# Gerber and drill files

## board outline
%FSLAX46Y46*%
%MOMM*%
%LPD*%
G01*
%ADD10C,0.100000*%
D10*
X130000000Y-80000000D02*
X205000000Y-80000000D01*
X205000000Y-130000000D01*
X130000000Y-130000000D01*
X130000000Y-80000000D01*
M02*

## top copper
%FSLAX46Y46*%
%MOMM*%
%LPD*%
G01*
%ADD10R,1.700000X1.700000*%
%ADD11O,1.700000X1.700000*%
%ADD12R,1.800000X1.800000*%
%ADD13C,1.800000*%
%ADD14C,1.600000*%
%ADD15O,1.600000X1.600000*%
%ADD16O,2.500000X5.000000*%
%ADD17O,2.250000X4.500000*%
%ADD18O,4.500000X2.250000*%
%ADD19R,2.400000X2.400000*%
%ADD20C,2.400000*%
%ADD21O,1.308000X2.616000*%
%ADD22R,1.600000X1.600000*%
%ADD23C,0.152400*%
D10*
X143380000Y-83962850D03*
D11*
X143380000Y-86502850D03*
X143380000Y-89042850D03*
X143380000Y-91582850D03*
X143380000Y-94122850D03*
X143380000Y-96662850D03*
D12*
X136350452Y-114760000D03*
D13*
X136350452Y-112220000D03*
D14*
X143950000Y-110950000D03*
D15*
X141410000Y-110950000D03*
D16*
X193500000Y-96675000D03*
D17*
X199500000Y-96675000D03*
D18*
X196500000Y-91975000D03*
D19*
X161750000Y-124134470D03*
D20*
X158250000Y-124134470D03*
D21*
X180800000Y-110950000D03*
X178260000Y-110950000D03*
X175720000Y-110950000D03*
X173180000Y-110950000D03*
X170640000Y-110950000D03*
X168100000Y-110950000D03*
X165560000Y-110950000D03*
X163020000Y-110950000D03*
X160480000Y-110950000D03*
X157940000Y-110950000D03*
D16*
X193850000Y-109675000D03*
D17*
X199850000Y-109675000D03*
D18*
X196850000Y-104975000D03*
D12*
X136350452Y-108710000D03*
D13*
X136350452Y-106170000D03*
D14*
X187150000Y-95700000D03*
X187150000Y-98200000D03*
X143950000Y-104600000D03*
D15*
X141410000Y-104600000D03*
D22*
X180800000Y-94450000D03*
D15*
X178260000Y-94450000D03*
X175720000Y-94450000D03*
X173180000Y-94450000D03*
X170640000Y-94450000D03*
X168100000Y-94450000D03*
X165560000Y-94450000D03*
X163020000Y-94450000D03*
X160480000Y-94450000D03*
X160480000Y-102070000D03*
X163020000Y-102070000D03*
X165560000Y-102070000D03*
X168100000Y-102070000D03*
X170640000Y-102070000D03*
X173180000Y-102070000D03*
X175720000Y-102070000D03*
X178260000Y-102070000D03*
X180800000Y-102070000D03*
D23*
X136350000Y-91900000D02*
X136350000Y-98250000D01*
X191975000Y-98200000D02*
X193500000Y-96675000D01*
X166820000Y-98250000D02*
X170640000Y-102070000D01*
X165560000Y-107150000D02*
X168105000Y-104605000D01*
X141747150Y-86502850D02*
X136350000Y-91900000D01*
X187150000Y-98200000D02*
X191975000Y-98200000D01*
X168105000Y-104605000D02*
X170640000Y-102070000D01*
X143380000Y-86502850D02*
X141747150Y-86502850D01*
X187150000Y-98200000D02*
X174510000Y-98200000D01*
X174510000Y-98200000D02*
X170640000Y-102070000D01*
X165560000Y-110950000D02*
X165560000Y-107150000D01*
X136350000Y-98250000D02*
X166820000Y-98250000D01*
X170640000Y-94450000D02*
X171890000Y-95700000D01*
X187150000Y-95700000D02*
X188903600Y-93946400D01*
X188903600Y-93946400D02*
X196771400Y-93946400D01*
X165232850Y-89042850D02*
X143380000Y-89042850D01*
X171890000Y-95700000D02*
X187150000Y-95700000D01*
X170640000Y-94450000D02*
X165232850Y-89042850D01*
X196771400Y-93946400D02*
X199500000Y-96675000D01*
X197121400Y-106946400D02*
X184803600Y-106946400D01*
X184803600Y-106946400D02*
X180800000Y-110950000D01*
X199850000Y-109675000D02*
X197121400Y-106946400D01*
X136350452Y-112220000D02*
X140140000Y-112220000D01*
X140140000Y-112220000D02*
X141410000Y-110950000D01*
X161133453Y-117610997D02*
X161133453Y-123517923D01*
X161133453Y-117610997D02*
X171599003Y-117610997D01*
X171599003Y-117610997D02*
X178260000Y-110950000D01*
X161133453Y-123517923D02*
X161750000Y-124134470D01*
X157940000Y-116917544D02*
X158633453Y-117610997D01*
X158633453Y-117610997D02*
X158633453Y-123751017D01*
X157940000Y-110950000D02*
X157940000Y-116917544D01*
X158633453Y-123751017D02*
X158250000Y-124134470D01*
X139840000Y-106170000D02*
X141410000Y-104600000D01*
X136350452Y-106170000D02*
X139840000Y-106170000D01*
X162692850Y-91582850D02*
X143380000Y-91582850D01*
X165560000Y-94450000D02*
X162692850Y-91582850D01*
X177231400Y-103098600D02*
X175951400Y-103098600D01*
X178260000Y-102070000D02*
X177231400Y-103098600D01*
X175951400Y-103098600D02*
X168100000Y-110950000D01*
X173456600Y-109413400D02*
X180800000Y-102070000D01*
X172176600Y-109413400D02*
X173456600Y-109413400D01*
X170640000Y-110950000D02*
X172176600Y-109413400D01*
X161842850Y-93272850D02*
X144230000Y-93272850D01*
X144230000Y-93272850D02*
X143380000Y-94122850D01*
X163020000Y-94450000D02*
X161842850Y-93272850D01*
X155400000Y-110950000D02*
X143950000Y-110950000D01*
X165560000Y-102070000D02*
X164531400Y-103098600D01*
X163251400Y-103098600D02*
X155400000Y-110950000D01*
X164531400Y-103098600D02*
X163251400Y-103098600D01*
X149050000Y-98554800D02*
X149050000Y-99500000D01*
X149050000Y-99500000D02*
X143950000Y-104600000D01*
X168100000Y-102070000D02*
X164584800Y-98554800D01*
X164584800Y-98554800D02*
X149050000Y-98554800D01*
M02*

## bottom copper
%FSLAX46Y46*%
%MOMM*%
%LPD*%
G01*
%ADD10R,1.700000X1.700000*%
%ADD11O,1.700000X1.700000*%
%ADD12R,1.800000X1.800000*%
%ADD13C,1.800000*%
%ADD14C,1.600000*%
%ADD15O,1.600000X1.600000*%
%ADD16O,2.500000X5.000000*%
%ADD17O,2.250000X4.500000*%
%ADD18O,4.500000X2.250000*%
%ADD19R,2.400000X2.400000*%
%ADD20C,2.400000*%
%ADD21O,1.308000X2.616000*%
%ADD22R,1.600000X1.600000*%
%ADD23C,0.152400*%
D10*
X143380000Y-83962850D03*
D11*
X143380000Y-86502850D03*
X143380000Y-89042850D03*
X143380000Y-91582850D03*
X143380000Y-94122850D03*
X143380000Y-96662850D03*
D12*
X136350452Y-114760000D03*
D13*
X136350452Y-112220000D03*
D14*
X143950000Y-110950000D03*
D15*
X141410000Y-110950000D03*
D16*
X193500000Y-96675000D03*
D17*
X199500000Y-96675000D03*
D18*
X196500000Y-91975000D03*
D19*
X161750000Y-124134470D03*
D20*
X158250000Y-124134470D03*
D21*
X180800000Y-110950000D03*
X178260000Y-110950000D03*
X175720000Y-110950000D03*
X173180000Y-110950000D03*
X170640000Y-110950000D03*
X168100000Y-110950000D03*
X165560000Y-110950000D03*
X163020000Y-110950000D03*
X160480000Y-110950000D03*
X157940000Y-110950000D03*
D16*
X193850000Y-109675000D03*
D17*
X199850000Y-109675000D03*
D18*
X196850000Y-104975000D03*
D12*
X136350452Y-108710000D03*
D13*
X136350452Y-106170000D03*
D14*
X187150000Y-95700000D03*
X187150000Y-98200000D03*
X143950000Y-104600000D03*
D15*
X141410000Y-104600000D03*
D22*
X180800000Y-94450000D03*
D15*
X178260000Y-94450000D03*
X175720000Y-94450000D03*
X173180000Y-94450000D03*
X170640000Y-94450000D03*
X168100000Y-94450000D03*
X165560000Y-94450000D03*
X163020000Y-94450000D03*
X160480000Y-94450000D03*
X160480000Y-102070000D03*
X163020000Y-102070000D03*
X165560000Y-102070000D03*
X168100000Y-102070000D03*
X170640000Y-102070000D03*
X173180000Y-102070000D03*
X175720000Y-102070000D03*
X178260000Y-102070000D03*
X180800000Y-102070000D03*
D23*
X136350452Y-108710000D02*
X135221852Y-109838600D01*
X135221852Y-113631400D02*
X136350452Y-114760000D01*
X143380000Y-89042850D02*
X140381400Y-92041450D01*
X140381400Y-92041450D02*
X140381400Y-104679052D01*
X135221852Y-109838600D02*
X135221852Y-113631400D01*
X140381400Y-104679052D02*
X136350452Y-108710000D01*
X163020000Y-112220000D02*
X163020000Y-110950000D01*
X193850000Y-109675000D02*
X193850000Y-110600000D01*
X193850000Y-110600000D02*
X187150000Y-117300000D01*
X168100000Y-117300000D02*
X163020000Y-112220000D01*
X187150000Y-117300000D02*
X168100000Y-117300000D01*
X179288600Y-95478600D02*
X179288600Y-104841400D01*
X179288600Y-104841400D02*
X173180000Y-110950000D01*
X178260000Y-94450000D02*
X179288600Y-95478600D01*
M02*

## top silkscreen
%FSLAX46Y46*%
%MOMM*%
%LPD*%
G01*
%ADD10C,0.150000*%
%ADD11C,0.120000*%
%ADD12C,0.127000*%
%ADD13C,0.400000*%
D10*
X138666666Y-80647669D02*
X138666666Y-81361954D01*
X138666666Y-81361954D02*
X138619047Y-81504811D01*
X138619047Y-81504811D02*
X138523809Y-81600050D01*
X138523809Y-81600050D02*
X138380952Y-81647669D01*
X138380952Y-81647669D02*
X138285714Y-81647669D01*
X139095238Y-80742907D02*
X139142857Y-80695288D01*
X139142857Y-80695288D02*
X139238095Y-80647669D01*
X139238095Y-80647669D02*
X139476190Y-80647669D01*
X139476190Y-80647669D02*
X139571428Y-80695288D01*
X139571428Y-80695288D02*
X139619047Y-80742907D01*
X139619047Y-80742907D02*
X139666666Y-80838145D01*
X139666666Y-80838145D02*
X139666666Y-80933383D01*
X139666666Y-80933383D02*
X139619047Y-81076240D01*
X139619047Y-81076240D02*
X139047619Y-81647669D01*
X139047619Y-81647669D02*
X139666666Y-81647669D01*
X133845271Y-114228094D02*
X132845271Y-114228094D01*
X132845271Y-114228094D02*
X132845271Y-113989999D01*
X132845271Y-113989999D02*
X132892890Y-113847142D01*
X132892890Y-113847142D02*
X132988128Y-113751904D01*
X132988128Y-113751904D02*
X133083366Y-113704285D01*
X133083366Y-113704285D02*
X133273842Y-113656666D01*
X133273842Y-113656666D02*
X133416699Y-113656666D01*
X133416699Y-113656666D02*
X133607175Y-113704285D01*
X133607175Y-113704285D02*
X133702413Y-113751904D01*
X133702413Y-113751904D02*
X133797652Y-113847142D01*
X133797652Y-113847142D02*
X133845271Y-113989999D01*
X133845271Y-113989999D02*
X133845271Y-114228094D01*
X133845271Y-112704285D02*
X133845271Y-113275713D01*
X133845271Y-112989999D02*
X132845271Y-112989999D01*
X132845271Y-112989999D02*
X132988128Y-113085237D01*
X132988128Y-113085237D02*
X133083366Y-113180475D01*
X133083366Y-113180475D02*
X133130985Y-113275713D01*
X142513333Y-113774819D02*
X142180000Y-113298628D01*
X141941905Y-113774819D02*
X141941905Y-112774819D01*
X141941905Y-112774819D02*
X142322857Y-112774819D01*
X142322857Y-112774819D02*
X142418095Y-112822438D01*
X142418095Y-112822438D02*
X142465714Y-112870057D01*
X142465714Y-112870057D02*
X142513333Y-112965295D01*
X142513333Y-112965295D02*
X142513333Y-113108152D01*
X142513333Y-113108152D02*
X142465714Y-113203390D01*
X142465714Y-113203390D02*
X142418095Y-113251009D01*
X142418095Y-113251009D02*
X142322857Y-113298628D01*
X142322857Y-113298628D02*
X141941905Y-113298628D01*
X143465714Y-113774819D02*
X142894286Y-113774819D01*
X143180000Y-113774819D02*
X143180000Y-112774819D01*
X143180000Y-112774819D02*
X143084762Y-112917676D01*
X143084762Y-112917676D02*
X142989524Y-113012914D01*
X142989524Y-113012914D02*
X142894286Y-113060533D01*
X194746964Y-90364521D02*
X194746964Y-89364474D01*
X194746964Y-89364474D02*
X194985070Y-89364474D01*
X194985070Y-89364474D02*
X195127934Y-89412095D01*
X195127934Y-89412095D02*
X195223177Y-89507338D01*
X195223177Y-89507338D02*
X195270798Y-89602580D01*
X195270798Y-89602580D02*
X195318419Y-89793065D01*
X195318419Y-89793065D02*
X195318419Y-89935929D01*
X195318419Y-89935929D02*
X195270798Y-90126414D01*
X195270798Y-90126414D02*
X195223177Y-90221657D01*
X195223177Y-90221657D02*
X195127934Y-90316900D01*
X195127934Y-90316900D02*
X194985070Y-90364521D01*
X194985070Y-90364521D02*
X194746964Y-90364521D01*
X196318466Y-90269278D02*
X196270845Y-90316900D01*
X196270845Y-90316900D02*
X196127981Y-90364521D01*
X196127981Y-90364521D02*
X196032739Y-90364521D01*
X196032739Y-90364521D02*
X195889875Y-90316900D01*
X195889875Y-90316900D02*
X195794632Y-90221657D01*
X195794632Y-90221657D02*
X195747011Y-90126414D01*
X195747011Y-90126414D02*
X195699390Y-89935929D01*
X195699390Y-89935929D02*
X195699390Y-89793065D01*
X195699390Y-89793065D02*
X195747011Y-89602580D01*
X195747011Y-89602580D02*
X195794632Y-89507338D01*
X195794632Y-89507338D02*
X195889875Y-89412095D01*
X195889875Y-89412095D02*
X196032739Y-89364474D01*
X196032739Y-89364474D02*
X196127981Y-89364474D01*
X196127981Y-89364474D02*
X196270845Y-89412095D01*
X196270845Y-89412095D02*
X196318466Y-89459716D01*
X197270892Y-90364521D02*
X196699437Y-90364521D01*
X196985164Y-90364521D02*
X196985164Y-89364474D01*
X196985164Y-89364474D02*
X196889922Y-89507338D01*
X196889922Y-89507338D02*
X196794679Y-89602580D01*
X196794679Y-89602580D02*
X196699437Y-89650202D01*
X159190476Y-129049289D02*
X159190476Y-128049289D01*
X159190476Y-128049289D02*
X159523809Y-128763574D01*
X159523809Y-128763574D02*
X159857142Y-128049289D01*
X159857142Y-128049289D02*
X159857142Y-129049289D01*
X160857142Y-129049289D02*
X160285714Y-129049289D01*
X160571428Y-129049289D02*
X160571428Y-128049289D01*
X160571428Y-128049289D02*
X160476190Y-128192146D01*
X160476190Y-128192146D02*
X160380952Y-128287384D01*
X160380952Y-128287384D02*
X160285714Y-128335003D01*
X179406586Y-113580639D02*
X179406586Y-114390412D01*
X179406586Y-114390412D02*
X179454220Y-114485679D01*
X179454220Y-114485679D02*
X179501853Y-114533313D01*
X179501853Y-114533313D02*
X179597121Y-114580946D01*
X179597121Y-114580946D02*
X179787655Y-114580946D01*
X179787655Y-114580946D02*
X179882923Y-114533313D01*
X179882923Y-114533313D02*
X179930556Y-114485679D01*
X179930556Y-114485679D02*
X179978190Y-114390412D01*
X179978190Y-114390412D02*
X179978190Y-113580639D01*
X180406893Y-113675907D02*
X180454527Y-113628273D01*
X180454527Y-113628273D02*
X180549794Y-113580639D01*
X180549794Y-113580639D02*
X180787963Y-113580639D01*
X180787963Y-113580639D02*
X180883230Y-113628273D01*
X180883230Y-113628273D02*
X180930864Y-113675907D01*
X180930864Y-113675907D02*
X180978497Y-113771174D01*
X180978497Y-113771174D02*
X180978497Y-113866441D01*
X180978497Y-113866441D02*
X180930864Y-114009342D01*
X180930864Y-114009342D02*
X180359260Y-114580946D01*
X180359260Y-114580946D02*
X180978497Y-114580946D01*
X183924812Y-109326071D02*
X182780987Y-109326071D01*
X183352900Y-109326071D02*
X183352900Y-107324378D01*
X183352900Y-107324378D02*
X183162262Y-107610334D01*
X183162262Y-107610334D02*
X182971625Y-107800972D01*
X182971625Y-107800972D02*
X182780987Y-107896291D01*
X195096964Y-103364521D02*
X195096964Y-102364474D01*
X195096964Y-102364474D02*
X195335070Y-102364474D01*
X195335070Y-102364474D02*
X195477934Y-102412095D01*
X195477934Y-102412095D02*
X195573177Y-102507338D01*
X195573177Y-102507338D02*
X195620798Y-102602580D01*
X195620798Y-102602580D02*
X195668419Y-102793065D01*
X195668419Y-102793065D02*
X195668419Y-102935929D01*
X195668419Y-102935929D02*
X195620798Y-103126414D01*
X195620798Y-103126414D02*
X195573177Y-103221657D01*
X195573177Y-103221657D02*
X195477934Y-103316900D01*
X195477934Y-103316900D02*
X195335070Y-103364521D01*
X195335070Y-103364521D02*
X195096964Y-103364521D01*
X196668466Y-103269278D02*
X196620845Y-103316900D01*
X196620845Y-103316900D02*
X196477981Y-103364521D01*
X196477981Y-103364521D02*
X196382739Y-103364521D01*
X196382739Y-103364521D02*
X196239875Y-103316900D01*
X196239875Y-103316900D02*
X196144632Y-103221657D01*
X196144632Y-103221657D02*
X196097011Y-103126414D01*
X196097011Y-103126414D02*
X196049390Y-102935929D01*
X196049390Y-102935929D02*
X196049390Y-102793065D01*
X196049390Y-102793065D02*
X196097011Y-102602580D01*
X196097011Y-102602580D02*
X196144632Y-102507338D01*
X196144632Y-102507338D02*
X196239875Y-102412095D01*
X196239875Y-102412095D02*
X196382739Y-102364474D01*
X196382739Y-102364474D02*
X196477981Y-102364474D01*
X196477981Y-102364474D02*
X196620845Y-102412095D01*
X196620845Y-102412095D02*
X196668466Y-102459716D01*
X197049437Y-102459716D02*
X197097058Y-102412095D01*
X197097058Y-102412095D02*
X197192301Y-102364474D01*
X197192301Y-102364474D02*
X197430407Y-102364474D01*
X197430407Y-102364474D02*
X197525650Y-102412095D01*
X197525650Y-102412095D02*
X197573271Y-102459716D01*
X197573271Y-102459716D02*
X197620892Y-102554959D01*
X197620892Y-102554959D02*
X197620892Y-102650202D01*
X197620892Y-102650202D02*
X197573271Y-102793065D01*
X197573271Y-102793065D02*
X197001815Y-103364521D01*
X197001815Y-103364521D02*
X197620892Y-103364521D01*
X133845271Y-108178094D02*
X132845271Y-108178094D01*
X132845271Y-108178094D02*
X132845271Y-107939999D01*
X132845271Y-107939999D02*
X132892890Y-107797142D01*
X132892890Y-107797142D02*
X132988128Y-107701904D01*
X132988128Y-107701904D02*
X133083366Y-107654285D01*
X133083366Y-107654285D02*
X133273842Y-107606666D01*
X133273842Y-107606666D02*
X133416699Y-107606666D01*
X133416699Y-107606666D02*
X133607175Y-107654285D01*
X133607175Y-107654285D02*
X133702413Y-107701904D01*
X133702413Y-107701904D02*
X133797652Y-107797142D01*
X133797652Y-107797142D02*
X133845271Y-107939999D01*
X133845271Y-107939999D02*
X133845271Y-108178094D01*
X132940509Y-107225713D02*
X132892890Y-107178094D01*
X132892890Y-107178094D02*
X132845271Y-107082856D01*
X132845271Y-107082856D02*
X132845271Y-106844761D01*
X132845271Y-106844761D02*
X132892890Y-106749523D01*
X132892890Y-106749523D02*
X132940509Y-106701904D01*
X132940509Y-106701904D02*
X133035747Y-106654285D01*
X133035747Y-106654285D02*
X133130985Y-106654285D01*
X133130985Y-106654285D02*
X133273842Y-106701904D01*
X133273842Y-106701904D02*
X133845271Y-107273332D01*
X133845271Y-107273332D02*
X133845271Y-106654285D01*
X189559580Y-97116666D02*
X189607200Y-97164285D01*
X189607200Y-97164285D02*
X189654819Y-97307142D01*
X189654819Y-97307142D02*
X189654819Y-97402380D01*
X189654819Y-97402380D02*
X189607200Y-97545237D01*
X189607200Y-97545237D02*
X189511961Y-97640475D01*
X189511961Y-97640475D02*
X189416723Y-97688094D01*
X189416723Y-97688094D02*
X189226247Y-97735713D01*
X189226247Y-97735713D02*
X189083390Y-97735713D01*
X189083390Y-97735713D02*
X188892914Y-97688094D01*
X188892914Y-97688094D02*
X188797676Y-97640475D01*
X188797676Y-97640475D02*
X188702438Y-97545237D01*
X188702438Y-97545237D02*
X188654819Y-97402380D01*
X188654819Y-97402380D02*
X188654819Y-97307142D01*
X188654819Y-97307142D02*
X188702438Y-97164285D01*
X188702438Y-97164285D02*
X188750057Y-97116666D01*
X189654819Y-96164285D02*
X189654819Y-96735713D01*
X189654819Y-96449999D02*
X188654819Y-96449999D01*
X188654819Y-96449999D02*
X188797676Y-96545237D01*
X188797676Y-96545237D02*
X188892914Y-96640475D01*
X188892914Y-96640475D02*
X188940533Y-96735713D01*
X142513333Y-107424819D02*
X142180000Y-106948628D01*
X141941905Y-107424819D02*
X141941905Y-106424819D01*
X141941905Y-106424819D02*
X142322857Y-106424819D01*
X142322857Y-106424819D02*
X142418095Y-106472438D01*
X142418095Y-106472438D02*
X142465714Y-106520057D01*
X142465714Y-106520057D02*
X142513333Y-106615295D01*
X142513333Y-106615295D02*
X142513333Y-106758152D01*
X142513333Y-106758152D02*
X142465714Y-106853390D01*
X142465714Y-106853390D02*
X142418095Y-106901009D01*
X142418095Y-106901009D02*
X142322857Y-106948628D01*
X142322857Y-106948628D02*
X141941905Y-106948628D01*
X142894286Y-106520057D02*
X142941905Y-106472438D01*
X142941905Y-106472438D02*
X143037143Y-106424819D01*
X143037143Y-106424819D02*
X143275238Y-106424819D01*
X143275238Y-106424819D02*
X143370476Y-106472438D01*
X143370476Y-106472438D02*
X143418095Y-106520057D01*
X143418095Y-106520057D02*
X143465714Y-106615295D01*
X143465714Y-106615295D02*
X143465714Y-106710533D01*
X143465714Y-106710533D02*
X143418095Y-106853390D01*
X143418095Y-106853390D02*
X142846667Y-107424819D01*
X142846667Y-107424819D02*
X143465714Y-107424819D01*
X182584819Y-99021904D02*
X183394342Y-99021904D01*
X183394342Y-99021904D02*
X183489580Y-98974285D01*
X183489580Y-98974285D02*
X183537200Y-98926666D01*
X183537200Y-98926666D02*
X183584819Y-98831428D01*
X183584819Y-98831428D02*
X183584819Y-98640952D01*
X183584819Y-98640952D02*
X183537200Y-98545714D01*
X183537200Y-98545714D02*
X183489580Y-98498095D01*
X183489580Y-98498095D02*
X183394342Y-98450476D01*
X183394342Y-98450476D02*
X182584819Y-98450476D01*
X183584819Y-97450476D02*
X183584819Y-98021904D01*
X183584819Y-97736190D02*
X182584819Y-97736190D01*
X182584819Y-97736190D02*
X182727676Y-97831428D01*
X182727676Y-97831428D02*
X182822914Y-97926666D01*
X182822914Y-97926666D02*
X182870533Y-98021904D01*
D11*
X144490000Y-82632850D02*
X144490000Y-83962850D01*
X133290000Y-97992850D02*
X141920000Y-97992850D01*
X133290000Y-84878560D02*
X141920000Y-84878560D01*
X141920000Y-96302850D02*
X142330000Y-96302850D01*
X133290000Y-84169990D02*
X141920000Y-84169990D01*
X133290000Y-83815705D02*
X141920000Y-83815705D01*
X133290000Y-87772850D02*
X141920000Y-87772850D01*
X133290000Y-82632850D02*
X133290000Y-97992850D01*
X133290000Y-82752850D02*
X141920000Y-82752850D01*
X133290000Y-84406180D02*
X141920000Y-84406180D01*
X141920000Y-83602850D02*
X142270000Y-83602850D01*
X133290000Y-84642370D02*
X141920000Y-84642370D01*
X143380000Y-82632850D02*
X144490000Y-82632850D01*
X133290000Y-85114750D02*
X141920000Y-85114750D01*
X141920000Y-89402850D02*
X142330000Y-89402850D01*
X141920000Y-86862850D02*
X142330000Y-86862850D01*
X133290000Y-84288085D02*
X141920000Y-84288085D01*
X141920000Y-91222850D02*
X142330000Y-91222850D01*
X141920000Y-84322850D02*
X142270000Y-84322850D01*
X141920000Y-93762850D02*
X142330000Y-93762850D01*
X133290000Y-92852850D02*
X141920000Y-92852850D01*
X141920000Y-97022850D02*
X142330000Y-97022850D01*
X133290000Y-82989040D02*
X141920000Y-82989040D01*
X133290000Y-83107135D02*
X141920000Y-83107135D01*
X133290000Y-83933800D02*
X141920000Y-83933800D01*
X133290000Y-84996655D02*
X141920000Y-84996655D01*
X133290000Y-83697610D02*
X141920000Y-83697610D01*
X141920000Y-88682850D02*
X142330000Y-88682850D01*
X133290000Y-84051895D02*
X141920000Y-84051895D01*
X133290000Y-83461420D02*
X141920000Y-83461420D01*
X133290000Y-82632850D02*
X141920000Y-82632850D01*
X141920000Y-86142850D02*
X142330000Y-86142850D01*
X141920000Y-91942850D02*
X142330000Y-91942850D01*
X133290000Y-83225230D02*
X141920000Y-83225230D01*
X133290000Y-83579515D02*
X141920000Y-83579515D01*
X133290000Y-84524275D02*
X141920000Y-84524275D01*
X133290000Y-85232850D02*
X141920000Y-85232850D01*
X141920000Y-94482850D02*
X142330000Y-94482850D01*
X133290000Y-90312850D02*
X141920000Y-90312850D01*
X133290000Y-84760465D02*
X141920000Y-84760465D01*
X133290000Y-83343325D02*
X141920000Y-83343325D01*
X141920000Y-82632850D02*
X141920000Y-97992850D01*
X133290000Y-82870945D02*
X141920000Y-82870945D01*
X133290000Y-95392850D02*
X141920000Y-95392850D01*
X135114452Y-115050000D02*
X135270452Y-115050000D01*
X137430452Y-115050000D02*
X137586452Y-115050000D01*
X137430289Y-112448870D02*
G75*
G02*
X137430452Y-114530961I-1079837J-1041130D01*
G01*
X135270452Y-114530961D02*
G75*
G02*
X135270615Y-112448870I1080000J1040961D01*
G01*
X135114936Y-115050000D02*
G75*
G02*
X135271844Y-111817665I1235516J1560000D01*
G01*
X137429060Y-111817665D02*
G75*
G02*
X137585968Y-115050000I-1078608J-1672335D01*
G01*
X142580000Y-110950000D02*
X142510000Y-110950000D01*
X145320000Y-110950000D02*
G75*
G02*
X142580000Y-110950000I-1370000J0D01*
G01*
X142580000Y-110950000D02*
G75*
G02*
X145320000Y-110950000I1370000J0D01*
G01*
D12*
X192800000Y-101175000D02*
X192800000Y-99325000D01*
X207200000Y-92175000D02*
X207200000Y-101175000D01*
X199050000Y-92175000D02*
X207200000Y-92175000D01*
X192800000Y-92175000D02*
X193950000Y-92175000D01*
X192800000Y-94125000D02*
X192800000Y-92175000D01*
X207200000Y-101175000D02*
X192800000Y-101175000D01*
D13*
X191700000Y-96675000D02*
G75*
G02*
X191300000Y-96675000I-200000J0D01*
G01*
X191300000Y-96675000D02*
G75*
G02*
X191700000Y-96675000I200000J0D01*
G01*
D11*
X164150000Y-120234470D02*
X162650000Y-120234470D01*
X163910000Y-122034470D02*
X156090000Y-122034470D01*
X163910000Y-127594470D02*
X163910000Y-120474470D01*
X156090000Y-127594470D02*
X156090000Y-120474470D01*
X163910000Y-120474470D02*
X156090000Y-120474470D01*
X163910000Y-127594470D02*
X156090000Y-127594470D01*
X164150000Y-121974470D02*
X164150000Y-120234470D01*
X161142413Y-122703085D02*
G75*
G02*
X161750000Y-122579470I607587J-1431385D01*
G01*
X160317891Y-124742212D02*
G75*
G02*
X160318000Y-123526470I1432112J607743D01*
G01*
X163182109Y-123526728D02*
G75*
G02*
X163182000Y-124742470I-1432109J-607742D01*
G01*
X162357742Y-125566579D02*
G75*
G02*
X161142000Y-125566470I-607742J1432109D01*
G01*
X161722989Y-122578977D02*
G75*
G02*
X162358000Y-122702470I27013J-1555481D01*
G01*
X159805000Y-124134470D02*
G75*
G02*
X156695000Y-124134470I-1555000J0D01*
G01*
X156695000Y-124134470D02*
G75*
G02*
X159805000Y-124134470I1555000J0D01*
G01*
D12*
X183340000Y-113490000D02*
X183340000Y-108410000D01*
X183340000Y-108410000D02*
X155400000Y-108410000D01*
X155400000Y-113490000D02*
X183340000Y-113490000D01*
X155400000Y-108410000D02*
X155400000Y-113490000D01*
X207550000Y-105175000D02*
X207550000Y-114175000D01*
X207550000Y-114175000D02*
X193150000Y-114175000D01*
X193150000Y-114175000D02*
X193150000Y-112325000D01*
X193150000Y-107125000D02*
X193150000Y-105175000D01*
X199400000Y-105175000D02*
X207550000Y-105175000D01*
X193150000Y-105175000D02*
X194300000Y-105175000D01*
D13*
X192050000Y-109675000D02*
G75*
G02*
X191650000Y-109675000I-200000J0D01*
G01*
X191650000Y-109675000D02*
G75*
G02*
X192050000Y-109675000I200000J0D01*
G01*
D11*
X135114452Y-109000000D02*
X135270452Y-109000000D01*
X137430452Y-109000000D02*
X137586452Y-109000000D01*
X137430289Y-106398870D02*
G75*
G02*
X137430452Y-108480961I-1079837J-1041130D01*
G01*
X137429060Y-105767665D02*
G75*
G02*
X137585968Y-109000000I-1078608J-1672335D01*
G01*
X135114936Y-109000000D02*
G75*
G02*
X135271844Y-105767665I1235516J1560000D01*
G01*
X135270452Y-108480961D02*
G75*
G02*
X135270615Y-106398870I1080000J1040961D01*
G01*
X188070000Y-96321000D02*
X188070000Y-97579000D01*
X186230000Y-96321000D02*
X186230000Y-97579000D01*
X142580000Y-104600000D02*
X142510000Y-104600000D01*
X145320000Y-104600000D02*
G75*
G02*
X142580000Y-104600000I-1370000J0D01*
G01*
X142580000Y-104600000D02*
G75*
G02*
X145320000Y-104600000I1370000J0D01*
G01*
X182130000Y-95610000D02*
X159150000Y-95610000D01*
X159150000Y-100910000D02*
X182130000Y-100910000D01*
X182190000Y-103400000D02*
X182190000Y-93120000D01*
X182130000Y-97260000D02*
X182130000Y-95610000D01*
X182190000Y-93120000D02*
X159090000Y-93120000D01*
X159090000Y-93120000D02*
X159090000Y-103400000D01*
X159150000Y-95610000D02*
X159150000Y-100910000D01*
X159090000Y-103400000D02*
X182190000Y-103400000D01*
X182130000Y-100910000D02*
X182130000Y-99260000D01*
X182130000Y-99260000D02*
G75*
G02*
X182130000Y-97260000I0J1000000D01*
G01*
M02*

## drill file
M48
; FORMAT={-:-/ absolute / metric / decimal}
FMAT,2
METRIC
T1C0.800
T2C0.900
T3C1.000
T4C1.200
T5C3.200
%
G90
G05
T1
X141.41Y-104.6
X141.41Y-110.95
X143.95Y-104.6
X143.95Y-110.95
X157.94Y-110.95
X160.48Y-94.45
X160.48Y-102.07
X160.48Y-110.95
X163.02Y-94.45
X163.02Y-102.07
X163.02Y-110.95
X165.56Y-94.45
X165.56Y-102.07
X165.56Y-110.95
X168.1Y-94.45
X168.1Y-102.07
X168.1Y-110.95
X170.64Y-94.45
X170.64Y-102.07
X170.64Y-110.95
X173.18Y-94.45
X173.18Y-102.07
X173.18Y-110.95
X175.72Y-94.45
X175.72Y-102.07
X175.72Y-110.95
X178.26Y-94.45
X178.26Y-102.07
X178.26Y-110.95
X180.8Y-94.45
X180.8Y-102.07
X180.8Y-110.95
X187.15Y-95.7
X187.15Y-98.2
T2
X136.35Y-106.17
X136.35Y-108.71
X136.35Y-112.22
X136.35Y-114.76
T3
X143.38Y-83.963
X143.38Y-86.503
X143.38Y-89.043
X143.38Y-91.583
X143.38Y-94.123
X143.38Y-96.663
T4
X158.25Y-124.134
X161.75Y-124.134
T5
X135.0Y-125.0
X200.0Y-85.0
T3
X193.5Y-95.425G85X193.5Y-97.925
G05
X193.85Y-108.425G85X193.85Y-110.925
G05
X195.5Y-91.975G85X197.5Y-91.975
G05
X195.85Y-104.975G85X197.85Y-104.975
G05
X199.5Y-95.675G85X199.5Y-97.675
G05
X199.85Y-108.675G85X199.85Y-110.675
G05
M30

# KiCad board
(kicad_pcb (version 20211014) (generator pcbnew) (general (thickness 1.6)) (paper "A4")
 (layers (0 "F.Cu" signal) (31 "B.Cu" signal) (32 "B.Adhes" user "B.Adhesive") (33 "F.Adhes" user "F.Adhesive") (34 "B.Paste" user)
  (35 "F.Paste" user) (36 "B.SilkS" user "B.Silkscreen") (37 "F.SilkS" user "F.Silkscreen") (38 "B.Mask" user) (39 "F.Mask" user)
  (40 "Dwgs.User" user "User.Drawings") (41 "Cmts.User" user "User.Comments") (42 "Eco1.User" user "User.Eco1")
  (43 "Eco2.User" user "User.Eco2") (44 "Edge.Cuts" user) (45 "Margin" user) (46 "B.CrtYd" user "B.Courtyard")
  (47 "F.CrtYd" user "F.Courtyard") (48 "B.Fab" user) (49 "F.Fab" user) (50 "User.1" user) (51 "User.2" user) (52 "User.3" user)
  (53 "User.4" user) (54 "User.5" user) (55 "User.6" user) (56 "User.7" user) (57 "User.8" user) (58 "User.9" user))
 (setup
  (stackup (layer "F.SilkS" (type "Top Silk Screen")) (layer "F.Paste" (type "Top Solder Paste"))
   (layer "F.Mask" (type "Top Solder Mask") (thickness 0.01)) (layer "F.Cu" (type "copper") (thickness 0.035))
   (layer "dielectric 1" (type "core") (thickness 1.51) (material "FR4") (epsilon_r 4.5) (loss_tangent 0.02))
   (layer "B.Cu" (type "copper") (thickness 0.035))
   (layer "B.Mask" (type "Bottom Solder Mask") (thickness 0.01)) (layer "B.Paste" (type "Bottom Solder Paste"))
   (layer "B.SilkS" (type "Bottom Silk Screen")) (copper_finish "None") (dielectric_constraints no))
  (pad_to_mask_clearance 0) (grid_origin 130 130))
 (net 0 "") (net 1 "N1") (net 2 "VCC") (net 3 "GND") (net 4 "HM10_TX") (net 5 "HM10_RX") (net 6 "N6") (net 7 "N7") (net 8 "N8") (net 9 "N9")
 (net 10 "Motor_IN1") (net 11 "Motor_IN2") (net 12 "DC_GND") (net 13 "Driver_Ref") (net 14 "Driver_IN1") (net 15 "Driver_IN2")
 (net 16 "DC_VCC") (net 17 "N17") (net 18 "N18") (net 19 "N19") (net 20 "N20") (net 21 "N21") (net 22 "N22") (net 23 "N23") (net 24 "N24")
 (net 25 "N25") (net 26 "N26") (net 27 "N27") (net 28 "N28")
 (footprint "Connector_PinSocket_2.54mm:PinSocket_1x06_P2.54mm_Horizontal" (layer "F.Cu") (at 143.38 83.96285)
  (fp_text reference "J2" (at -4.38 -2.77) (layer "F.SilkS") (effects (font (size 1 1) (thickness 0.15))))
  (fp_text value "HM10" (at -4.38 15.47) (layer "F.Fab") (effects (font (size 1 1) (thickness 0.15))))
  (fp_line (start 1.11 -1.33) (end 1.11 0) (layer "F.SilkS") (width 0.12))
  (fp_line (start -10.09 14.03) (end -1.46 14.03) (layer "F.SilkS") (width 0.12))
  (fp_line (start -10.09 0.91571) (end -1.46 0.91571) (layer "F.SilkS") (width 0.12))
  (fp_line (start -1.46 12.34) (end -1.05 12.34) (layer "F.SilkS") (width 0.12))
  (fp_line (start -10.09 0.20714) (end -1.46 0.20714) (layer "F.SilkS") (width 0.12))
  (fp_line (start -10.09 -0.147145) (end -1.46 -0.147145) (layer "F.SilkS") (width 0.12))
  (fp_line (start -10.09 3.81) (end -1.46 3.81) (layer "F.SilkS") (width 0.12))
  (fp_line (start -10.09 -1.33) (end -10.09 14.03) (layer "F.SilkS") (width 0.12))
  (fp_line (start -10.09 -1.21) (end -1.46 -1.21) (layer "F.SilkS") (width 0.12))
  (fp_line (start -10.09 0.44333) (end -1.46 0.44333) (layer "F.SilkS") (width 0.12))
  (fp_line (start -1.46 -0.36) (end -1.11 -0.36) (layer "F.SilkS") (width 0.12))
  (fp_line (start -10.09 0.67952) (end -1.46 0.67952) (layer "F.SilkS") (width 0.12))
  (fp_line (start 0 -1.33) (end 1.11 -1.33) (layer "F.SilkS") (width 0.12))
  (fp_line (start -10.09 1.1519) (end -1.46 1.1519) (layer "F.SilkS") (width 0.12))
  (fp_line (start -1.46 5.44) (end -1.05 5.44) (layer "F.SilkS") (width 0.12))
  (fp_line (start -1.46 2.9) (end -1.05 2.9) (layer "F.SilkS") (width 0.12))
  (fp_line (start -10.09 0.325235) (end -1.46 0.325235) (layer "F.SilkS") (width 0.12))
  (fp_line (start -1.46 7.26) (end -1.05 7.26) (layer "F.SilkS") (width 0.12))
  (fp_line (start -1.46 0.36) (end -1.11 0.36) (layer "F.SilkS") (width 0.12))
  (fp_line (start -1.46 9.8) (end -1.05 9.8) (layer "F.SilkS") (width 0.12))
  (fp_line (start -10.09 8.89) (end -1.46 8.89) (layer "F.SilkS") (width 0.12))
  (fp_line (start -1.46 13.06) (end -1.05 13.06) (layer "F.SilkS") (width 0.12))
  (fp_line (start -10.09 -0.97381) (end -1.46 -0.97381) (layer "F.SilkS") (width 0.12))
  (fp_line (start -10.09 -0.855715) (end -1.46 -0.855715) (layer "F.SilkS") (width 0.12))
  (fp_line (start -10.09 -0.02905) (end -1.46 -0.02905) (layer "F.SilkS") (width 0.12))
  (fp_line (start -10.09 1.033805) (end -1.46 1.033805) (layer "F.SilkS") (width 0.12))
  (fp_line (start -10.09 -0.26524) (end -1.46 -0.26524) (layer "F.SilkS") (width 0.12))
  (fp_line (start -1.46 4.72) (end -1.05 4.72) (layer "F.SilkS") (width 0.12))
  (fp_line (start -10.09 0.089045) (end -1.46 0.089045) (layer "F.SilkS") (width 0.12))
  (fp_line (start -10.09 -0.50143) (end -1.46 -0.50143) (layer "F.SilkS") (width 0.12))
  (fp_line (start -10.09 -1.33) (end -1.46 -1.33) (layer "F.SilkS") (width 0.12))
  (fp_line (start -1.46 2.18) (end -1.05 2.18) (layer "F.SilkS") (width 0.12))
  (fp_line (start -1.46 7.98) (end -1.05 7.98) (layer "F.SilkS") (width 0.12))
  (fp_line (start -10.09 -0.73762) (end -1.46 -0.73762) (layer "F.SilkS") (width 0.12))
  (fp_line (start -10.09 -0.383335) (end -1.46 -0.383335) (layer "F.SilkS") (width 0.12))
  (fp_line (start -10.09 0.561425) (end -1.46 0.561425) (layer "F.SilkS") (width 0.12))
  (fp_line (start -10.09 1.27) (end -1.46 1.27) (layer "F.SilkS") (width 0.12))
  (fp_line (start -1.46 10.52) (end -1.05 10.52) (layer "F.SilkS") (width 0.12))
  (fp_line (start -10.09 6.35) (end -1.46 6.35) (layer "F.SilkS") (width 0.12))
  (fp_line (start -10.09 0.797615) (end -1.46 0.797615) (layer "F.SilkS") (width 0.12))
  (fp_line (start -10.09 -0.619525) (end -1.46 -0.619525) (layer "F.SilkS") (width 0.12))
  (fp_line (start -1.46 -1.33) (end -1.46 14.03) (layer "F.SilkS") (width 0.12))
  (fp_line (start -10.09 -1.091905) (end -1.46 -1.091905) (layer "F.SilkS") (width 0.12))
  (fp_line (start -10.09 11.43) (end -1.46 11.43) (layer "F.SilkS") (width 0.12))
  (pad "1" thru_hole rect (at 0 0) (size 1.7 1.7) (drill 1) (layers *.Cu *.Mask) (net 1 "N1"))
  (pad "2" thru_hole oval (at 0 2.54) (size 1.7 1.7) (drill 1) (layers *.Cu *.Mask) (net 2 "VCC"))
  (pad "3" thru_hole oval (at 0 5.08) (size 1.7 1.7) (drill 1) (layers *.Cu *.Mask) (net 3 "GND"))
  (pad "4" thru_hole oval (at 0 7.62) (size 1.7 1.7) (drill 1) (layers *.Cu *.Mask) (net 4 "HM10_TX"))
  (pad "5" thru_hole oval (at 0 10.16) (size 1.7 1.7) (drill 1) (layers *.Cu *.Mask) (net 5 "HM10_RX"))
  (pad "6" thru_hole oval (at 0 12.7) (size 1.7 1.7) (drill 1) (layers *.Cu *.Mask) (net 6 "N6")))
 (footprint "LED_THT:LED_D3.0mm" (layer "F.Cu") (at 136.350452 114.76 90)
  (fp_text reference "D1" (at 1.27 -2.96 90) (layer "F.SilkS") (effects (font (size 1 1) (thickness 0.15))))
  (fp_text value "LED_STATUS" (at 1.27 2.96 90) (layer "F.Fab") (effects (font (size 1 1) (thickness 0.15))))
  (fp_line (start -0.29 -1.236) (end -0.29 -1.08) (layer "F.SilkS") (width 0.12))
  (fp_line (start -0.29 1.08) (end -0.29 1.236) (layer "F.SilkS") (width 0.12))
  (fp_arc (start 2.31113 1.079837) (mid 1.270117 1.5) (end 0.229039 1.08) (layer "F.SilkS") (width 0.12))
  (fp_arc (start 0.229039 -1.08) (mid 1.270117 -1.5) (end 2.31113 -1.079837) (layer "F.SilkS") (width 0.12))
  (fp_arc (start -0.29 -1.235516) (mid 1.366487 -1.987659) (end 2.942335 -1.078608) (layer "F.SilkS") (width 0.12))
  (fp_arc (start 2.942335 1.078608) (mid 1.366487 1.987659) (end -0.29 1.235516) (layer "F.SilkS") (width 0.12))
  (pad "1" thru_hole rect (at 0 0 90) (size 1.8 1.8) (drill 0.9) (layers *.Cu *.Mask) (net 3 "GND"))
  (pad "2" thru_hole circle (at 2.54 0 90) (size 1.8 1.8) (drill 0.9) (layers *.Cu *.Mask) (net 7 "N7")))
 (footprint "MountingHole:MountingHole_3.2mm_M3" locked (layer "F.Cu") (at 200 85)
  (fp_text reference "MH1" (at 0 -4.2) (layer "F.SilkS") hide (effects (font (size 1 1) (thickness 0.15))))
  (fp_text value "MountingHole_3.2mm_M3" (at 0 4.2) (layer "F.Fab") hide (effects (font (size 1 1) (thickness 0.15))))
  (pad "" np_thru_hole circle locked (at 0 0) (size 3.2 3.2) (drill 3.2) (layers *.Cu *.Mask)))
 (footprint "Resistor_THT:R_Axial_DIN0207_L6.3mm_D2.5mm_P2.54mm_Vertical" (layer "F.Cu") (at 143.95 110.95 180)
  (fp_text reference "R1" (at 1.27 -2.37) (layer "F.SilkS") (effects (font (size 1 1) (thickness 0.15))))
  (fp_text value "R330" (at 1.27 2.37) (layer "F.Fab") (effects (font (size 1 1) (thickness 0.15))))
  (fp_line (start 1.37 0) (end 1.44 0) (layer "F.SilkS") (width 0.12))
  (fp_circle (center 0 0) (end 1.37 0) (layer "F.SilkS") (width 0.12) (fill none))
  (pad "1" thru_hole circle (at 0 0 180) (size 1.6 1.6) (drill 0.8) (layers *.Cu *.Mask) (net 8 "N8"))
  (pad "2" thru_hole oval (at 2.54 0 180) (size 1.6 1.6) (drill 0.8) (layers *.Cu *.Mask) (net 7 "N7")))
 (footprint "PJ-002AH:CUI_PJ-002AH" (layer "F.Cu") (at 193.5 96.675)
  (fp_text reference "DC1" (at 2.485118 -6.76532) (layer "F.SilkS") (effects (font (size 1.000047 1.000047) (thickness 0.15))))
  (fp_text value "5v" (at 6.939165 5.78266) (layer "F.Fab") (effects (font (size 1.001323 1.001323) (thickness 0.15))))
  (fp_line (start -0.7 4.5) (end -0.7 2.65) (layer "F.SilkS") (width 0.127))
  (fp_line (start 13.7 -4.5) (end 13.7 4.5) (layer "F.SilkS") (width 0.127))
  (fp_line (start 5.55 -4.5) (end 13.7 -4.5) (layer "F.SilkS") (width 0.127))
  (fp_line (start -0.7 -4.5) (end 0.45 -4.5) (layer "F.SilkS") (width 0.127))
  (fp_line (start -0.7 -2.55) (end -0.7 -4.5) (layer "F.SilkS") (width 0.127))
  (fp_line (start 13.7 4.5) (end -0.7 4.5) (layer "F.SilkS") (width 0.127))
  (fp_circle (center -2 0) (end -1.8 0) (layer "F.SilkS") (width 0.4) (fill none))
  (pad "1" thru_hole oval locked (at 0 0) (size 2.5 5) (drill oval 1 3.5) (layers *.Cu *.Mask) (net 2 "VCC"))
  (pad "2" thru_hole oval locked (at 6 0) (size 2.25 4.5) (drill oval 1 3) (layers *.Cu *.Mask) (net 3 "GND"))
  (pad "3" thru_hole oval locked (at 3 -4.7) (size 4.5 2.25) (drill oval 3 1) (layers *.Cu *.Mask) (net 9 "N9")))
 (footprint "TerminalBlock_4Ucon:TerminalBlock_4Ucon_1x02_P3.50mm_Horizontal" (layer "F.Cu") (at 161.75 124.13447 180)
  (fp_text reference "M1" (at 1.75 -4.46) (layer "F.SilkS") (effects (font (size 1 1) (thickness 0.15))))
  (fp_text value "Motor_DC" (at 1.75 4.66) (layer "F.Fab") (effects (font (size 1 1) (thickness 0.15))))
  (fp_line (start -2.4 3.9) (end -0.9 3.9) (layer "F.SilkS") (width 0.12))
  (fp_line (start -2.16 2.1) (end 5.66 2.1) (layer "F.SilkS") (width 0.12))
  (fp_line (start -2.16 -3.46) (end -2.16 3.66) (layer "F.SilkS") (width 0.12))
  (fp_line (start 5.66 -3.46) (end 5.66 3.66) (layer "F.SilkS") (width 0.12))
  (fp_line (start -2.16 3.66) (end 5.66 3.66) (layer "F.SilkS") (width 0.12))
  (fp_line (start -2.16 -3.46) (end 5.66 -3.46) (layer "F.SilkS") (width 0.12))
  (fp_line (start -2.4 2.16) (end -2.4 3.9) (layer "F.SilkS") (width 0.12))
  (fp_arc (start 0.607587 1.431385) (mid 0.310017 1.523783) (end 0 1.555) (layer "F.SilkS") (width 0.12))
  (fp_arc (start 1.432109 -0.607742) (mid 1.555727 0.00014) (end 1.432 0.608) (layer "F.SilkS") (width 0.12))
  (fp_arc (start -1.432109 0.607742) (mid -1.555727 -0.00014) (end -1.432 -0.608) (layer "F.SilkS") (width 0.12))
  (fp_arc (start -0.607742 -1.432109) (mid 0.00014 -1.555727) (end 0.608 -1.432) (layer "F.SilkS") (width 0.12))
  (fp_arc (start 0.027011 1.555493) (mid -0.296984 1.527118) (end -0.608 1.432) (layer "F.SilkS") (width 0.12))
  (fp_circle (center 3.5 0) (end 5.055 0) (layer "F.SilkS") (width 0.12) (fill none))
  (pad "1" thru_hole rect (at 0 0 180) (size 2.4 2.4) (drill 1.2) (layers *.Cu *.Mask) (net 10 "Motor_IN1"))
  (pad "2" thru_hole circle (at 3.5 0 180) (size 2.4 2.4) (drill 1.2) (layers *.Cu *.Mask) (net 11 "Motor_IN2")))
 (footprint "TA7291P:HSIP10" (layer "F.Cu") (at 168.1 110.95 180)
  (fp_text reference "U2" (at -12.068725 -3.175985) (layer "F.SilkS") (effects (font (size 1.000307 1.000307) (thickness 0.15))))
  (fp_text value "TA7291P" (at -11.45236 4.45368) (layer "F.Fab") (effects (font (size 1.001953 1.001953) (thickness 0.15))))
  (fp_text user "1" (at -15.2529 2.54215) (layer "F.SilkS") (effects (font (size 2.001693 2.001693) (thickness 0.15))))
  (fp_line (start -15.24 -2.54) (end -15.24 2.54) (layer "F.SilkS") (width 0.127))
  (fp_line (start -15.24 2.54) (end 12.7 2.54) (layer "F.SilkS") (width 0.127))
  (fp_line (start 12.7 -2.54) (end -15.24 -2.54) (layer "F.SilkS") (width 0.127))
  (fp_line (start 12.7 2.54) (end 12.7 -2.54) (layer "F.SilkS") (width 0.127))
  (pad "1" thru_hole oval locked (at -12.7 0 180) (size 1.308 2.616) (drill 0.8) (layers *.Cu *.Mask) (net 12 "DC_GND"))
  (pad "2" thru_hole oval locked (at -10.16 0 180) (size 1.308 2.616) (drill 0.8) (layers *.Cu *.Mask) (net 10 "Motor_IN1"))
  (pad "3" thru_hole oval locked (at -7.62 0 180) (size 1.308 2.616) (drill 0.8) (layers *.Cu *.Mask))
  (pad "4" thru_hole oval locked (at -5.08 0 180) (size 1.308 2.616) (drill 0.8) (layers *.Cu *.Mask) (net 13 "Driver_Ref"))
  (pad "5" thru_hole oval locked (at -2.54 0 180) (size 1.308 2.616) (drill 0.8) (layers *.Cu *.Mask) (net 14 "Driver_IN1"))
  (pad "6" thru_hole oval locked (at 0 0 180) (size 1.308 2.616) (drill 0.8) (layers *.Cu *.Mask) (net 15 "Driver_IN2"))
  (pad "7" thru_hole oval locked (at 2.54 0 180) (size 1.308 2.616) (drill 0.8) (layers *.Cu *.Mask) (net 2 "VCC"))
  (pad "8" thru_hole oval locked (at 5.08 0 180) (size 1.308 2.616) (drill 0.8) (layers *.Cu *.Mask) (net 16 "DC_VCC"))
  (pad "9" thru_hole oval locked (at 7.62 0 180) (size 1.308 2.616) (drill 0.8) (layers *.Cu *.Mask))
  (pad "10" thru_hole oval locked (at 10.16 0 180) (size 1.308 2.616) (drill 0.8) (layers *.Cu *.Mask) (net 11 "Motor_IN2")))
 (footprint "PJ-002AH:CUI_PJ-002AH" (layer "F.Cu") (at 193.85 109.675)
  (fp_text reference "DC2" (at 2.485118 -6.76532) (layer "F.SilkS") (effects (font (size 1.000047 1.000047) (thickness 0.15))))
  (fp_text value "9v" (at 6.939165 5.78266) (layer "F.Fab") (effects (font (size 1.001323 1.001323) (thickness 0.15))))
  (fp_line (start 13.7 -4.5) (end 13.7 4.5) (layer "F.SilkS") (width 0.127))
  (fp_line (start 13.7 4.5) (end -0.7 4.5) (layer "F.SilkS") (width 0.127))
  (fp_line (start -0.7 4.5) (end -0.7 2.65) (layer "F.SilkS") (width 0.127))
  (fp_line (start -0.7 -2.55) (end -0.7 -4.5) (layer "F.SilkS") (width 0.127))
  (fp_line (start 5.55 -4.5) (end 13.7 -4.5) (layer "F.SilkS") (width 0.127))
  (fp_line (start -0.7 -4.5) (end 0.45 -4.5) (layer "F.SilkS") (width 0.127))
  (fp_circle (center -2 0) (end -1.8 0) (layer "F.SilkS") (width 0.4) (fill none))
  (pad "1" thru_hole oval locked (at 0 0) (size 2.5 5) (drill oval 1 3.5) (layers *.Cu *.Mask) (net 16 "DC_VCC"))
  (pad "2" thru_hole oval locked (at 6 0) (size 2.25 4.5) (drill oval 1 3) (layers *.Cu *.Mask) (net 12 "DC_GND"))
  (pad "3" thru_hole oval locked (at 3 -4.7) (size 4.5 2.25) (drill oval 3 1) (layers *.Cu *.Mask) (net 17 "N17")))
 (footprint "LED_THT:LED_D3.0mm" (layer "F.Cu") (at 136.350452 108.71 90)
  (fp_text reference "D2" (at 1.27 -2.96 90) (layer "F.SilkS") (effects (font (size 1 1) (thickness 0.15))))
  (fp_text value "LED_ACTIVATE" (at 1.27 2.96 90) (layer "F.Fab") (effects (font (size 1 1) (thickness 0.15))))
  (fp_line (start -0.29 -1.236) (end -0.29 -1.08) (layer "F.SilkS") (width 0.12))
  (fp_line (start -0.29 1.08) (end -0.29 1.236) (layer "F.SilkS") (width 0.12))
  (fp_arc (start 2.31113 1.079837) (mid 1.270117 1.5) (end 0.229039 1.08) (layer "F.SilkS") (width 0.12))
  (fp_arc (start 2.942335 1.078608) (mid 1.366487 1.987659) (end -0.29 1.235516) (layer "F.SilkS") (width 0.12))
  (fp_arc (start -0.29 -1.235516) (mid 1.366487 -1.987659) (end 2.942335 -1.078608) (layer "F.SilkS") (width 0.12))
  (fp_arc (start 0.229039 -1.08) (mid 1.270117 -1.5) (end 2.31113 -1.079837) (layer "F.SilkS") (width 0.12))
  (pad "1" thru_hole rect (at 0 0 90) (size 1.8 1.8) (drill 0.9) (layers *.Cu *.Mask) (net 3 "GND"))
  (pad "2" thru_hole circle (at 2.54 0 90) (size 1.8 1.8) (drill 0.9) (layers *.Cu *.Mask) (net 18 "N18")))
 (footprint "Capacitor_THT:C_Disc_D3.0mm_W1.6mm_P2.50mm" (layer "F.Cu") (at 187.15 95.7 -90)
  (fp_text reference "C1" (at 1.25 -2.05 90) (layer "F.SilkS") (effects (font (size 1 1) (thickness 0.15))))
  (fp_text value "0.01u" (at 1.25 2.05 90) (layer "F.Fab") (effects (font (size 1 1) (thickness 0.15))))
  (fp_line (start 0.621 -0.92) (end 1.879 -0.92) (layer "F.SilkS") (width 0.12))
  (fp_line (start 0.621 0.92) (end 1.879 0.92) (layer "F.SilkS") (width 0.12))
  (pad "1" thru_hole circle (at 0 0 270) (size 1.6 1.6) (drill 0.8) (layers *.Cu *.Mask) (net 3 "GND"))
  (pad "2" thru_hole circle (at 2.5 0 270) (size 1.6 1.6) (drill 0.8) (layers *.Cu *.Mask) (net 2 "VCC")))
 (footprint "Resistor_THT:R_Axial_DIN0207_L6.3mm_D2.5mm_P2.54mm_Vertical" (layer "F.Cu") (at 143.95 104.6 180)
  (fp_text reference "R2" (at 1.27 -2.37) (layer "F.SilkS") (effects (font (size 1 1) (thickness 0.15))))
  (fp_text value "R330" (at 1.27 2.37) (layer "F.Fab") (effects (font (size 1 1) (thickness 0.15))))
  (fp_line (start 1.37 0) (end 1.44 0) (layer "F.SilkS") (width 0.12))
  (fp_circle (center 0 0) (end 1.37 0) (layer "F.SilkS") (width 0.12) (fill none))
  (pad "1" thru_hole circle (at 0 0 180) (size 1.6 1.6) (drill 0.8) (layers *.Cu *.Mask) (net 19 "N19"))
  (pad "2" thru_hole oval (at 2.54 0 180) (size 1.6 1.6) (drill 0.8) (layers *.Cu *.Mask) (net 18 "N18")))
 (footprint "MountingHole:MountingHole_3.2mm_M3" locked (layer "F.Cu") (at 135 125)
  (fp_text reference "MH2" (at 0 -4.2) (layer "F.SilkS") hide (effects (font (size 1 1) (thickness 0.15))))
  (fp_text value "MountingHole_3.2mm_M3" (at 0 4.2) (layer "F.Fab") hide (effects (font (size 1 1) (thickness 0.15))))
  (pad "" np_thru_hole circle locked (at 0 0) (size 3.2 3.2) (drill 3.2) (layers *.Cu *.Mask)))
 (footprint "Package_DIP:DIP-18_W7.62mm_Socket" (layer "F.Cu") (at 180.8 94.45 -90)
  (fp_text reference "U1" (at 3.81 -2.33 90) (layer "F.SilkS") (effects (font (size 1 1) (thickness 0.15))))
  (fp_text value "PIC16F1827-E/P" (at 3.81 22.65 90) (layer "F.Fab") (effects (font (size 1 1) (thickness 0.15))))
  (fp_line (start 1.16 -1.33) (end 1.16 21.65) (layer "F.SilkS") (width 0.12))
  (fp_line (start 6.46 21.65) (end 6.46 -1.33) (layer "F.SilkS") (width 0.12))
  (fp_line (start 8.95 -1.39) (end -1.33 -1.39) (layer "F.SilkS") (width 0.12))
  (fp_line (start 2.81 -1.33) (end 1.16 -1.33) (layer "F.SilkS") (width 0.12))
  (fp_line (start -1.33 -1.39) (end -1.33 21.71) (layer "F.SilkS") (width 0.12))
  (fp_line (start -1.33 21.71) (end 8.95 21.71) (layer "F.SilkS") (width 0.12))
  (fp_line (start 1.16 21.65) (end 6.46 21.65) (layer "F.SilkS") (width 0.12))
  (fp_line (start 8.95 21.71) (end 8.95 -1.39) (layer "F.SilkS") (width 0.12))
  (fp_line (start 6.46 -1.33) (end 4.81 -1.33) (layer "F.SilkS") (width 0.12))
  (fp_arc (start 4.81 -1.33) (mid 3.81 -0.33) (end 2.81 -1.33) (layer "F.SilkS") (width 0.12))
  (pad "1" thru_hole rect (at 0 0 270) (size 1.6 1.6) (drill 0.8) (layers *.Cu *.Mask) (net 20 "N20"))
  (pad "2" thru_hole oval (at 0 2.54 270) (size 1.6 1.6) (drill 0.8) (layers *.Cu *.Mask) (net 13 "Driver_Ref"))
  (pad "3" thru_hole oval (at 0 5.08 270) (size 1.6 1.6) (drill 0.8) (layers *.Cu *.Mask) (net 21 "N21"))
  (pad "4" thru_hole oval (at 0 7.62 270) (size 1.6 1.6) (drill 0.8) (layers *.Cu *.Mask) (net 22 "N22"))
  (pad "5" thru_hole oval (at 0 10.16 270) (size 1.6 1.6) (drill 0.8) (layers *.Cu *.Mask) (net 3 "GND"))
  (pad "6" thru_hole oval (at 0 12.7 270) (size 1.6 1.6) (drill 0.8) (layers *.Cu *.Mask) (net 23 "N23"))
  (pad "7" thru_hole oval (at 0 15.24 270) (size 1.6 1.6) (drill 0.8) (layers *.Cu *.Mask) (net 4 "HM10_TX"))
  (pad "8" thru_hole oval (at 0 17.78 270) (size 1.6 1.6) (drill 0.8) (layers *.Cu *.Mask) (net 5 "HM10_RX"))
  (pad "9" thru_hole oval (at 0 20.32 270) (size 1.6 1.6) (drill 0.8) (layers *.Cu *.Mask) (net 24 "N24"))
  (pad "10" thru_hole oval (at 7.62 20.32 270) (size 1.6 1.6) (drill 0.8) (layers *.Cu *.Mask) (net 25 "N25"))
  (pad "11" thru_hole oval (at 7.62 17.78 270) (size 1.6 1.6) (drill 0.8) (layers *.Cu *.Mask) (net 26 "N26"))
  (pad "12" thru_hole oval (at 7.62 15.24 270) (size 1.6 1.6) (drill 0.8) (layers *.Cu *.Mask) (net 8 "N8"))
  (pad "13" thru_hole oval (at 7.62 12.7 270) (size 1.6 1.6) (drill 0.8) (layers *.Cu *.Mask) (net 19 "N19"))
  (pad "14" thru_hole oval (at 7.62 10.16 270) (size 1.6 1.6) (drill 0.8) (layers *.Cu *.Mask) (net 2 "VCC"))
  (pad "15" thru_hole oval (at 7.62 7.62 270) (size 1.6 1.6) (drill 0.8) (layers *.Cu *.Mask) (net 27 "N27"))
  (pad "16" thru_hole oval (at 7.62 5.08 270) (size 1.6 1.6) (drill 0.8) (layers *.Cu *.Mask) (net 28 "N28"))
  (pad "17" thru_hole oval (at 7.62 2.54 270) (size 1.6 1.6) (drill 0.8) (layers *.Cu *.Mask) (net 15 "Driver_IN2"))
  (pad "18" thru_hole oval (at 7.62 0 270) (size 1.6 1.6) (drill 0.8) (layers *.Cu *.Mask) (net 14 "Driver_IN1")))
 (gr_rect locked (start 130 130) (end 205 80) (layer "Edge.Cuts") (width 0.1) (fill none))
 (segment (start 136.35 91.9) (end 136.35 98.25) (width 0.1524) (layer "F.Cu") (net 2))
 (segment (start 191.975 98.2) (end 193.5 96.675) (width 0.1524) (layer "F.Cu") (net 2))
 (segment (start 166.82 98.25) (end 170.64 102.07) (width 0.1524) (layer "F.Cu") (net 2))
 (segment (start 165.56 107.15) (end 168.105 104.605) (width 0.1524) (layer "F.Cu") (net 2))
 (segment (start 141.74715 86.50285) (end 136.35 91.9) (width 0.1524) (layer "F.Cu") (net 2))
 (segment (start 187.15 98.2) (end 191.975 98.2) (width 0.1524) (layer "F.Cu") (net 2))
 (segment (start 168.105 104.605) (end 170.64 102.07) (width 0.1524) (layer "F.Cu") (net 2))
 (segment (start 143.38 86.50285) (end 141.74715 86.50285) (width 0.1524) (layer "F.Cu") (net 2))
 (segment (start 187.15 98.2) (end 174.51 98.2) (width 0.1524) (layer "F.Cu") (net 2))
 (segment (start 174.51 98.2) (end 170.64 102.07) (width 0.1524) (layer "F.Cu") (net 2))
 (segment (start 165.56 110.95) (end 165.56 107.15) (width 0.1524) (layer "F.Cu") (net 2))
 (segment (start 136.35 98.25) (end 166.82 98.25) (width 0.1524) (layer "F.Cu") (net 2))
 (segment (start 170.64 94.45) (end 171.89 95.7) (width 0.1524) (layer "F.Cu") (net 3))
 (segment (start 187.15 95.7) (end 188.9036 93.9464) (width 0.1524) (layer "F.Cu") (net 3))
 (segment (start 188.9036 93.9464) (end 196.7714 93.9464) (width 0.1524) (layer "F.Cu") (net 3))
 (segment (start 165.23285 89.04285) (end 143.38 89.04285) (width 0.1524) (layer "F.Cu") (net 3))
 (segment (start 171.89 95.7) (end 187.15 95.7) (width 0.1524) (layer "F.Cu") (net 3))
 (segment (start 170.64 94.45) (end 165.23285 89.04285) (width 0.1524) (layer "F.Cu") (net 3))
 (segment (start 196.7714 93.9464) (end 199.5 96.675) (width 0.1524) (layer "F.Cu") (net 3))
 (segment (start 136.350452 108.71) (end 135.221852 109.8386) (width 0.1524) (layer "B.Cu") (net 3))
 (segment (start 135.221852 113.6314) (end 136.350452 114.76) (width 0.1524) (layer "B.Cu") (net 3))
 (segment (start 143.38 89.04285) (end 140.3814 92.04145) (width 0.1524) (layer "B.Cu") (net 3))
 (segment (start 140.3814 92.04145) (end 140.3814 104.679052) (width 0.1524) (layer "B.Cu") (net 3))
 (segment (start 135.221852 109.8386) (end 135.221852 113.6314) (width 0.1524) (layer "B.Cu") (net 3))
 (segment (start 140.3814 104.679052) (end 136.350452 108.71) (width 0.1524) (layer "B.Cu") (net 3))
 (segment (start 163.02 112.22) (end 163.02 110.95) (width 0.1524) (layer "B.Cu") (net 16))
 (segment (start 193.85 109.675) (end 193.85 110.6) (width 0.1524) (layer "B.Cu") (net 16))
 (segment (start 193.85 110.6) (end 187.15 117.3) (width 0.1524) (layer "B.Cu") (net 16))
 (segment (start 168.1 117.3) (end 163.02 112.22) (width 0.1524) (layer "B.Cu") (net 16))
 (segment (start 187.15 117.3) (end 168.1 117.3) (width 0.1524) (layer "B.Cu") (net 16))
 (segment (start 197.1214 106.9464) (end 184.8036 106.9464) (width 0.1524) (layer "F.Cu") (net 12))
 (segment (start 184.8036 106.9464) (end 180.8 110.95) (width 0.1524) (layer "F.Cu") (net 12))
 (segment (start 199.85 109.675) (end 197.1214 106.9464) (width 0.1524) (layer "F.Cu") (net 12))
 (segment (start 136.350452 112.22) (end 140.14 112.22) (width 0.1524) (layer "F.Cu") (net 7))
 (segment (start 140.14 112.22) (end 141.41 110.95) (width 0.1524) (layer "F.Cu") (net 7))
 (segment (start 161.133453 117.610997) (end 161.133453 123.517923) (width 0.1524) (layer "F.Cu") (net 10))
 (segment (start 161.133453 117.610997) (end 171.599003 117.610997) (width 0.1524) (layer "F.Cu") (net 10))
 (segment (start 171.599003 117.610997) (end 178.26 110.95) (width 0.1524) (layer "F.Cu") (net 10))
 (segment (start 161.133453 123.517923) (end 161.75 124.13447) (width 0.1524) (layer "F.Cu") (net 10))
 (segment (start 157.94 116.917544) (end 158.633453 117.610997) (width 0.1524) (layer "F.Cu") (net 11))
 (segment (start 158.633453 117.610997) (end 158.633453 123.751017) (width 0.1524) (layer "F.Cu") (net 11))
 (segment (start 157.94 110.95) (end 157.94 116.917544) (width 0.1524) (layer "F.Cu") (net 11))
 (segment (start 158.633453 123.751017) (end 158.25 124.13447) (width 0.1524) (layer "F.Cu") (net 11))
 (segment (start 139.84 106.17) (end 141.41 104.6) (width 0.1524) (layer "F.Cu") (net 18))
 (segment (start 136.350452 106.17) (end 139.84 106.17) (width 0.1524) (layer "F.Cu") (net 18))
 (segment (start 162.69285 91.58285) (end 143.38 91.58285) (width 0.1524) (layer "F.Cu") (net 4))
 (segment (start 165.56 94.45) (end 162.69285 91.58285) (width 0.1524) (layer "F.Cu") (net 4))
 (segment (start 179.2886 95.4786) (end 179.2886 104.8414) (width 0.1524) (layer "B.Cu") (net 13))
 (segment (start 179.2886 104.8414) (end 173.18 110.95) (width 0.1524) (layer "B.Cu") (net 13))
 (segment (start 178.26 94.45) (end 179.2886 95.4786) (width 0.1524) (layer "B.Cu") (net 13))
 (segment (start 177.2314 103.0986) (end 175.9514 103.0986) (width 0.1524) (layer "F.Cu") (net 15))
 (segment (start 178.26 102.07) (end 177.2314 103.0986) (width 0.1524) (layer "F.Cu") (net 15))
 (segment (start 175.9514 103.0986) (end 168.1 110.95) (width 0.1524) (layer "F.Cu") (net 15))
 (segment (start 173.4566 109.4134) (end 180.8 102.07) (width 0.1524) (layer "F.Cu") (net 14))
 (segment (start 172.1766 109.4134) (end 173.4566 109.4134) (width 0.1524) (layer "F.Cu") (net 14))
 (segment (start 170.64 110.95) (end 172.1766 109.4134) (width 0.1524) (layer "F.Cu") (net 14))
 (segment (start 161.84285 93.27285) (end 144.23 93.27285) (width 0.1524) (layer "F.Cu") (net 5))
 (segment (start 144.23 93.27285) (end 143.38 94.12285) (width 0.1524) (layer "F.Cu") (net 5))
 (segment (start 163.02 94.45) (end 161.84285 93.27285) (width 0.1524) (layer "F.Cu") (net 5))
 (segment (start 155.4 110.95) (end 143.95 110.95) (width 0.1524) (layer "F.Cu") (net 8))
 (segment (start 165.56 102.07) (end 164.5314 103.0986) (width 0.1524) (layer "F.Cu") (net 8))
 (segment (start 163.2514 103.0986) (end 155.4 110.95) (width 0.1524) (layer "F.Cu") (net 8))
 (segment (start 164.5314 103.0986) (end 163.2514 103.0986) (width 0.1524) (layer "F.Cu") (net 8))
 (segment (start 149.05 98.5548) (end 149.05 99.5) (width 0.1524) (layer "F.Cu") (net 19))
 (segment (start 149.05 99.5) (end 143.95 104.6) (width 0.1524) (layer "F.Cu") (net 19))
 (segment (start 168.1 102.07) (end 164.5848 98.5548) (width 0.1524) (layer "F.Cu") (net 19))
 (segment (start 164.5848 98.5548) (end 149.05 98.5548) (width 0.1524) (layer "F.Cu") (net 19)))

